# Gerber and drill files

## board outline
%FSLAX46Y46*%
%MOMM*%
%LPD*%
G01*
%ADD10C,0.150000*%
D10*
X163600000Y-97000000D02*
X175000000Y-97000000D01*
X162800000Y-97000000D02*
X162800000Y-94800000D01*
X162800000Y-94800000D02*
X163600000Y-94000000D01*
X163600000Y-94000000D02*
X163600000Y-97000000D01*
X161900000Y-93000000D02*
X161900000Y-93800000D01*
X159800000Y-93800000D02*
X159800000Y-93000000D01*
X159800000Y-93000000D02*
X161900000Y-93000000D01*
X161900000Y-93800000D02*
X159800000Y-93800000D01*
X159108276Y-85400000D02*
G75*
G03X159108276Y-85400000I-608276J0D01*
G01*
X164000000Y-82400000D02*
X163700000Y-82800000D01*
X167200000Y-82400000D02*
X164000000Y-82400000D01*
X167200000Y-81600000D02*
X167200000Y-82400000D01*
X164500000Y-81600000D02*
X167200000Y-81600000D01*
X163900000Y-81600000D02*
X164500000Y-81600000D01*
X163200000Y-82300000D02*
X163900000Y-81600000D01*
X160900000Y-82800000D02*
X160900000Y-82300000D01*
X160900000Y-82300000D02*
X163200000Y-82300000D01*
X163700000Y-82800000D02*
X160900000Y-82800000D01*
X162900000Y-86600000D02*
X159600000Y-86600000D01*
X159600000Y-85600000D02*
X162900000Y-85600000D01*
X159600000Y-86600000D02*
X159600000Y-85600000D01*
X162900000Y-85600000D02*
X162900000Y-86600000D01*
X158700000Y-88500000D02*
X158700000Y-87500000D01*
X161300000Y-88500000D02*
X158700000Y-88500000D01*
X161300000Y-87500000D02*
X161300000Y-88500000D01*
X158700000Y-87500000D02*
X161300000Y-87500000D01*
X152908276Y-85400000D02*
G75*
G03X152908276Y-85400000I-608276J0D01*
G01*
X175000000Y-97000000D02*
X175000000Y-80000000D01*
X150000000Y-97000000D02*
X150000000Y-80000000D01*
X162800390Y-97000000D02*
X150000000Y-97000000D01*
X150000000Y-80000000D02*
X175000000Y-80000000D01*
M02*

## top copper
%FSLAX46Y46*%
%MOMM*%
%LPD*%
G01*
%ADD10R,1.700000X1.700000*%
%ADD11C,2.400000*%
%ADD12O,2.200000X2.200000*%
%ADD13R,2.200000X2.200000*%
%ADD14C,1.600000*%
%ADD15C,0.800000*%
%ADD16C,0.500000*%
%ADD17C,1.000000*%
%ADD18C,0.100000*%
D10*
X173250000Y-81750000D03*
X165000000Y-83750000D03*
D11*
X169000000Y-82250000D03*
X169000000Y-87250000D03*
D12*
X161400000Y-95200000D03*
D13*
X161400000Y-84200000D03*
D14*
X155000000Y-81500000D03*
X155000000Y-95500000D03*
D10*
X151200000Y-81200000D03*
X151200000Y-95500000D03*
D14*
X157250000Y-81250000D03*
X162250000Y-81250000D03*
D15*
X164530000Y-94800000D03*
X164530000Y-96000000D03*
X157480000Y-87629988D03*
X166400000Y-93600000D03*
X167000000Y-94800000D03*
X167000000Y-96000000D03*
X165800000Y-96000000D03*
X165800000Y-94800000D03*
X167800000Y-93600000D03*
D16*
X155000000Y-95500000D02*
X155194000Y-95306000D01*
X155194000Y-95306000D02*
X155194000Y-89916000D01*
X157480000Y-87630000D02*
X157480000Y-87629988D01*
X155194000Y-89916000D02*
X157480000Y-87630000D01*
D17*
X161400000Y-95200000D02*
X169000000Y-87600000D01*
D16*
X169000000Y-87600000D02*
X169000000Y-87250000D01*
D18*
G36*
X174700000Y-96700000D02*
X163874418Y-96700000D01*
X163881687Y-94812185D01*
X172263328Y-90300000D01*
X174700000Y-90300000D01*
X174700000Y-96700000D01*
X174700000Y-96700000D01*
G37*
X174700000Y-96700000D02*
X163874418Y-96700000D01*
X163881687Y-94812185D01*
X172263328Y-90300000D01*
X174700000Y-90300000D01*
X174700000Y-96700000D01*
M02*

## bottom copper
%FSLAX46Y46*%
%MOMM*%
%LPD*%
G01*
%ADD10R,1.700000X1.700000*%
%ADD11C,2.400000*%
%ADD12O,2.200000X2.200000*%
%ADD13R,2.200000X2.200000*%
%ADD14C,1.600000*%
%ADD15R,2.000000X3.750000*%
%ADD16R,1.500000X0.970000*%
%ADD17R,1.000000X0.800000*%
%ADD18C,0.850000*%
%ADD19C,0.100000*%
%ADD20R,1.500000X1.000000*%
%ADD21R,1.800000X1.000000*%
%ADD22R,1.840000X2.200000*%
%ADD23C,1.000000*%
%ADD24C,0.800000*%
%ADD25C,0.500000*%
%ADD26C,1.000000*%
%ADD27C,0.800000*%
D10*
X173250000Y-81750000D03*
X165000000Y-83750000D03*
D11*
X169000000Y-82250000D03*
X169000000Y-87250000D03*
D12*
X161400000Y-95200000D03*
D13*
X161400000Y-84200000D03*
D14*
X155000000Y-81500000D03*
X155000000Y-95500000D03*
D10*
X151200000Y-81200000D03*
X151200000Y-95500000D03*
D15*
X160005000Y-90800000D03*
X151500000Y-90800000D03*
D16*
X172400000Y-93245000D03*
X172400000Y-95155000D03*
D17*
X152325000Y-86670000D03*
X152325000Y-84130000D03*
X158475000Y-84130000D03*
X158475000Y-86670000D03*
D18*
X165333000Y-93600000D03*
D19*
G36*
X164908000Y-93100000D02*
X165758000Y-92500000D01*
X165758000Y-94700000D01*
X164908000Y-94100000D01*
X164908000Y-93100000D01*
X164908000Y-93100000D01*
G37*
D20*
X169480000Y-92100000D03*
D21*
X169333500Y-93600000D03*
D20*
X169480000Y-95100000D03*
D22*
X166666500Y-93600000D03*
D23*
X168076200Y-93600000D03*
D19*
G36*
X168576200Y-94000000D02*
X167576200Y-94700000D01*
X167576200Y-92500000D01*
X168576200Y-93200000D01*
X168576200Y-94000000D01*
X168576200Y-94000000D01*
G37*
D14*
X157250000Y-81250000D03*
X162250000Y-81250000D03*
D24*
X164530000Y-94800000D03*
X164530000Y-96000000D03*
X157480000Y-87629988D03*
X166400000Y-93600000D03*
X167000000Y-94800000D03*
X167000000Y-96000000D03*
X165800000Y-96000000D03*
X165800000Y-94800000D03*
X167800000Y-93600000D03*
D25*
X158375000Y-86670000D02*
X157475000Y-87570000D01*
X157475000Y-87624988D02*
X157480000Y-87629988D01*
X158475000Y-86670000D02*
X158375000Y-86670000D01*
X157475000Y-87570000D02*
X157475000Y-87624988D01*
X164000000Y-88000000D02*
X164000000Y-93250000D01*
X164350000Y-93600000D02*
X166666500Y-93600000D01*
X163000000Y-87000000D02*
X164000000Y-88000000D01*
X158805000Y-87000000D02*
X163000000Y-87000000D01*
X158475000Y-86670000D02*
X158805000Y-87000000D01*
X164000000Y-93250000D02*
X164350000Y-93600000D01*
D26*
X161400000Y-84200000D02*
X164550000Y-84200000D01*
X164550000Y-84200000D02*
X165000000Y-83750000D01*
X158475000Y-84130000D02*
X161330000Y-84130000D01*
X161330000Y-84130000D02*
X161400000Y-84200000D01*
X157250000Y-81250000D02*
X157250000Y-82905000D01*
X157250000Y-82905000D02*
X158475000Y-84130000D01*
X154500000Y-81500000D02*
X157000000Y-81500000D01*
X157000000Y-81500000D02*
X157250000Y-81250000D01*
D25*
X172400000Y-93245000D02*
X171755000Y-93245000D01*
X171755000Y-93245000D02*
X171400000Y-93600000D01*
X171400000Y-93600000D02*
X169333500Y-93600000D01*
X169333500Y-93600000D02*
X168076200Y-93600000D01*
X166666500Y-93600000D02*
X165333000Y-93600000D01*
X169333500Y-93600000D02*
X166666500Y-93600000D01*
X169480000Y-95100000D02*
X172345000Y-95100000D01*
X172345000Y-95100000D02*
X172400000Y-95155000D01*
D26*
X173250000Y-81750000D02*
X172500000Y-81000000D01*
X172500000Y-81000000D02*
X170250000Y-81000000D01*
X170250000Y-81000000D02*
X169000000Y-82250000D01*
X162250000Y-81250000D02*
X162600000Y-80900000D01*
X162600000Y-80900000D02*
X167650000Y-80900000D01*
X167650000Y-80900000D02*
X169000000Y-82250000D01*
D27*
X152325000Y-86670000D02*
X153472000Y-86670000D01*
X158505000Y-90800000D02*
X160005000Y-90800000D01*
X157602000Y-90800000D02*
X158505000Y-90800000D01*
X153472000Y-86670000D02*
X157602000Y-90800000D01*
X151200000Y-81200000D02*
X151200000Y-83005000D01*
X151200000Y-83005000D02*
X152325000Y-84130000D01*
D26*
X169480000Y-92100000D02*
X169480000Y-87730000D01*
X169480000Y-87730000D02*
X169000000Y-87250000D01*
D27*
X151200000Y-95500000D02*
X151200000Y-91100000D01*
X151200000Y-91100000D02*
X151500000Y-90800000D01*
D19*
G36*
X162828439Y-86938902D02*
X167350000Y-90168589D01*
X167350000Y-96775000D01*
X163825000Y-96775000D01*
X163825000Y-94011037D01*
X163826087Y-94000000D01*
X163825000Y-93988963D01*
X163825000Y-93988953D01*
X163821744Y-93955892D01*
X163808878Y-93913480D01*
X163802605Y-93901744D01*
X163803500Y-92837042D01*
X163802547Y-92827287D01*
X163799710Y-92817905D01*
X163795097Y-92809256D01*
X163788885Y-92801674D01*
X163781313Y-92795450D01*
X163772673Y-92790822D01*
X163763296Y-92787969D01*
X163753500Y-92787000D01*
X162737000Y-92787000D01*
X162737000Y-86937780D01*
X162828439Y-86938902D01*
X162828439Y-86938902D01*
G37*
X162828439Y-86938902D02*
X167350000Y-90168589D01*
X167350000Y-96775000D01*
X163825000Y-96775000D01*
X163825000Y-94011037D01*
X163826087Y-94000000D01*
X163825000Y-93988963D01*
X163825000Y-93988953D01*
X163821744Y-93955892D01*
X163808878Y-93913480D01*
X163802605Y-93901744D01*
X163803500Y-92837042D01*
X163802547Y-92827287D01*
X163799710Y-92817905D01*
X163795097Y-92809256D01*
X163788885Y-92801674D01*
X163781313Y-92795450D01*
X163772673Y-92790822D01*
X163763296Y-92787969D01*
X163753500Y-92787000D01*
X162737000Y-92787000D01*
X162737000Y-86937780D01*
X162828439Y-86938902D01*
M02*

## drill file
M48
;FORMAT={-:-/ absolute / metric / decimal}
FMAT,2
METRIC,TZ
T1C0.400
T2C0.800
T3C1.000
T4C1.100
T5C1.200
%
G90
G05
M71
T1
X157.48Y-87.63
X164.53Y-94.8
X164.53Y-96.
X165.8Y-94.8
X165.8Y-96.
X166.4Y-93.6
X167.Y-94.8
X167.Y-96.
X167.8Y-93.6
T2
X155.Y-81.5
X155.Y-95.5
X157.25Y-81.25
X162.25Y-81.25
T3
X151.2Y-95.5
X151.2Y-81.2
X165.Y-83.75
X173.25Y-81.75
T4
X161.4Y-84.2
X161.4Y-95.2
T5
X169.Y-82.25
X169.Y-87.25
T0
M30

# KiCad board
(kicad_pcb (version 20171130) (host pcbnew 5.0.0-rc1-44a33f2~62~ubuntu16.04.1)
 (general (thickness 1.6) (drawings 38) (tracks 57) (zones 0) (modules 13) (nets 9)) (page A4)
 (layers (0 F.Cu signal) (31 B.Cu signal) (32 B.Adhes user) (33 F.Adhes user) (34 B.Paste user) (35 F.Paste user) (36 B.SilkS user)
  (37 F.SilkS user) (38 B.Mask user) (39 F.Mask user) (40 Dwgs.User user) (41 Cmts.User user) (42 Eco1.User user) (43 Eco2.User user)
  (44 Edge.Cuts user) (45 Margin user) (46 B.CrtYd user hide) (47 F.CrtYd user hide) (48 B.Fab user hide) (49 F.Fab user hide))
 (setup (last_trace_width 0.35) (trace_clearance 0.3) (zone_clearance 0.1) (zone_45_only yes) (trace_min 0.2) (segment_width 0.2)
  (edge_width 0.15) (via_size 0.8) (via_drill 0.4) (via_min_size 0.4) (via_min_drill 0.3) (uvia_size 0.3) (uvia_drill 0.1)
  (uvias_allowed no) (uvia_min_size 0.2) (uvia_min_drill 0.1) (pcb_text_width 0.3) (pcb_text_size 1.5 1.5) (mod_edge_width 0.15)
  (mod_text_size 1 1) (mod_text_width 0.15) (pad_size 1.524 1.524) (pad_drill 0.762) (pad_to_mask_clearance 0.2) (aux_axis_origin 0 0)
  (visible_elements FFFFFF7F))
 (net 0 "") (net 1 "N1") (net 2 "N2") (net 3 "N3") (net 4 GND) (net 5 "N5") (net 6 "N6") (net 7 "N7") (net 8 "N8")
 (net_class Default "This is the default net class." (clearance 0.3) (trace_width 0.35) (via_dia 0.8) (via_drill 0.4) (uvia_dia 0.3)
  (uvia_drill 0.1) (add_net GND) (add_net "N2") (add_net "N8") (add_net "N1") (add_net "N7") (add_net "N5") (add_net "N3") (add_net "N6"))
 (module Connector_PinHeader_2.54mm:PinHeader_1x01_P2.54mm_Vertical (layer F.Cu) (at 173.25 81.75)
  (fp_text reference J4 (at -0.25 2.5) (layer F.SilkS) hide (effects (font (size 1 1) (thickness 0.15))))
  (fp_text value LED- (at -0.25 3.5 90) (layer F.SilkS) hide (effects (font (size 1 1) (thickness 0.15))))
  (pad 1 thru_hole rect (at 0 0) (size 1.7 1.7) (drill 1) (layers *.Cu *.Mask) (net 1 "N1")))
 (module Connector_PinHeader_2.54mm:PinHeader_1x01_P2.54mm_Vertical (layer F.Cu) (at 165 83.75)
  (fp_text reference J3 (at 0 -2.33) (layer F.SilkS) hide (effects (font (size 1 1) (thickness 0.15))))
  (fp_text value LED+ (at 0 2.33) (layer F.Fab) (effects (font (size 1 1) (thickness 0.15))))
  (pad 1 thru_hole rect (at 0 0) (size 1.7 1.7) (drill 1) (layers *.Cu *.Mask) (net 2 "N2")))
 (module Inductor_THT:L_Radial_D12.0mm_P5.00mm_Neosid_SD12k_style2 (layer F.Cu) (at 169 82.25 270)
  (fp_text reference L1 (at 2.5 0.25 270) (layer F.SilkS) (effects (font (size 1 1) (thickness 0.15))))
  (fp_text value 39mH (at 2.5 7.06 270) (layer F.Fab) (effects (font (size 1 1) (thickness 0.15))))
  (pad 1 thru_hole circle (at 0 0 270) (size 2.4 2.4) (drill 1.2) (layers *.Cu *.Mask) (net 1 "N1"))
  (pad 2 thru_hole circle (at 5 0 270) (size 2.4 2.4) (drill 1.2) (layers *.Cu *.Mask) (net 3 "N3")))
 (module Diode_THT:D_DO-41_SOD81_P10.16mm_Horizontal (layer F.Cu) (at 161.4 84.2 270)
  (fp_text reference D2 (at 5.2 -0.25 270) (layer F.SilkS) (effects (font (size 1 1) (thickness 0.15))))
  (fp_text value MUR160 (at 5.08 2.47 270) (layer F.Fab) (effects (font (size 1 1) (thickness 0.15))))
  (pad 2 thru_hole oval (at 11 0 270) (size 2.2 2.2) (drill 1.1) (layers *.Cu *.Mask) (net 3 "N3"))
  (pad 1 thru_hole rect (at 0 0 270) (size 2.2 2.2) (drill 1.1) (layers *.Cu *.Mask) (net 2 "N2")))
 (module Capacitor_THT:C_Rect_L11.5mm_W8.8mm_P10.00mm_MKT (layer F.Cu) (at 155 83.5 270)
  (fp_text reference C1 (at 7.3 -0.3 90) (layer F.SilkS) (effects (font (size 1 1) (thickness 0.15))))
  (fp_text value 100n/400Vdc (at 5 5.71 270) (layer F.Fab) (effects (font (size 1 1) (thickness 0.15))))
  (pad 1 thru_hole circle (at -2 0 270) (size 1.6 1.6) (drill 0.8) (layers *.Cu *.Mask) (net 2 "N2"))
  (pad 2 thru_hole circle (at 12 0 270) (size 1.6 1.6) (drill 0.8) (layers *.Cu *.Mask) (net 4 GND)))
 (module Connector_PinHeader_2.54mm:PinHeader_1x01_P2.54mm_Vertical (layer F.Cu) (at 151.2 81.2)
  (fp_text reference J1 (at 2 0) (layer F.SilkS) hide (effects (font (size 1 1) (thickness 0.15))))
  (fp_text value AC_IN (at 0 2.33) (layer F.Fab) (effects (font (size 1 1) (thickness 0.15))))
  (pad 1 thru_hole rect (at 0 0) (size 1.7 1.7) (drill 1) (layers *.Cu *.Mask) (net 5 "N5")))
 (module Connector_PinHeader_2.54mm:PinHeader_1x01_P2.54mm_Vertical (layer F.Cu) (at 151.2 95.5)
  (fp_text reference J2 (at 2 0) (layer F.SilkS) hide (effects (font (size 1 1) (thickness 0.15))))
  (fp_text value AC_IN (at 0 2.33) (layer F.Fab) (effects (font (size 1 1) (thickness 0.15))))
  (pad 1 thru_hole rect (at 0 0) (size 1.7 1.7) (drill 1) (layers *.Cu *.Mask) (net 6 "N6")))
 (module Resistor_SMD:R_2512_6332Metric (layer B.Cu) (at 157 90.8 180)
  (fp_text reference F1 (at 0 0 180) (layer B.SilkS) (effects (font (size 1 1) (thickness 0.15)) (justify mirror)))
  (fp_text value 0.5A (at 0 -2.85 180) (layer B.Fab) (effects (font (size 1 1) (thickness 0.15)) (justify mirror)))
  (pad 1 smd rect (at -3.005 0 180) (size 2 3.75) (layers B.Cu B.Paste B.Mask) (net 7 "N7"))
  (pad 2 smd rect (at 5.5 0 180) (size 2 3.75) (layers B.Cu B.Paste B.Mask) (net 6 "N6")))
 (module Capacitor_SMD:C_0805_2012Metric (layer B.Cu) (at 172.4 94.2 270)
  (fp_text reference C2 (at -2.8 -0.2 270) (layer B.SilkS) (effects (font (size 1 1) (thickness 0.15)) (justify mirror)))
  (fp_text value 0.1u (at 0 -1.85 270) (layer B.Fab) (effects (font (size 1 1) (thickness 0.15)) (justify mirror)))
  (pad 1 smd rect (at -0.955 0 270) (size 0.97 1.5) (layers B.Cu B.Paste B.Mask) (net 4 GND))
  (pad 2 smd rect (at 0.955 0 270) (size 0.97 1.5) (layers B.Cu B.Paste B.Mask) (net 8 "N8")))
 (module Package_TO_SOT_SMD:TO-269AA (layer B.Cu) (at 155.4 85.4)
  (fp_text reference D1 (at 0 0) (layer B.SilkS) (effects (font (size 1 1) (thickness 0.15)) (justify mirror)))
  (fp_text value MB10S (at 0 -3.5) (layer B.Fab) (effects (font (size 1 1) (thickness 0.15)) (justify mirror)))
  (pad 1 smd rect (at -3.075 1.27) (size 1 0.8) (layers B.Cu B.Paste B.Mask) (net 7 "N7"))
  (pad 2 smd rect (at -3.075 -1.27) (size 1 0.8) (layers B.Cu B.Paste B.Mask) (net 5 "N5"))
  (pad 3 smd rect (at 3.075 -1.27) (size 1 0.8) (layers B.Cu B.Paste B.Mask) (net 2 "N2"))
  (pad 4 smd rect (at 3.075 1.27) (size 1 0.8) (layers B.Cu B.Paste B.Mask) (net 4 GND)))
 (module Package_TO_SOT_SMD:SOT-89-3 (layer B.Cu) (at 168 93.6 180)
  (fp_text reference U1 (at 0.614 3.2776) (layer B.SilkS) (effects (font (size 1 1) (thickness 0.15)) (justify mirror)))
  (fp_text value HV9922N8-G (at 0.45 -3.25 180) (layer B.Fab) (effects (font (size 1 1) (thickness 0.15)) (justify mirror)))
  (pad 2 smd trapezoid (at 2.667 0 270) (size 1.6 0.85) (rect_delta 0 -0.6) (layers B.Cu B.Paste B.Mask) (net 4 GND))
  (pad 1 smd rect (at -1.48 1.5 270) (size 1 1.5) (layers B.Cu B.Paste B.Mask) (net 3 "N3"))
  (pad 2 smd rect (at -1.3335 0 270) (size 1 1.8) (layers B.Cu B.Paste B.Mask) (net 4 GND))
  (pad 3 smd rect (at -1.48 -1.5 270) (size 1 1.5) (layers B.Cu B.Paste B.Mask) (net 8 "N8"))
  (pad 2 smd rect (at 1.3335 0 270) (size 2.2 1.84) (layers B.Cu B.Paste B.Mask) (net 4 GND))
  (pad 2 smd trapezoid (at -0.0762 0 90) (size 1.5 1) (rect_delta 0 -0.7) (layers B.Cu B.Paste B.Mask) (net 4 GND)))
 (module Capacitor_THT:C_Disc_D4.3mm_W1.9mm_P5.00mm (layer F.Cu) (at 157.25 81.25)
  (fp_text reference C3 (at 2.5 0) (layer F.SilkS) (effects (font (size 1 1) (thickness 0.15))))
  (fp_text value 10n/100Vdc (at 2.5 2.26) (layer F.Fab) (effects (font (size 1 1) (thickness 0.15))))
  (pad 1 thru_hole circle (at 0 0) (size 1.6 1.6) (drill 0.8) (layers *.Cu *.Mask) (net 2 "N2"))
  (pad 2 thru_hole circle (at 5 0) (size 1.6 1.6) (drill 0.8) (layers *.Cu *.Mask) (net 1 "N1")))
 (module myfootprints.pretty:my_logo (layer F.Cu) (at 170.942 93.98)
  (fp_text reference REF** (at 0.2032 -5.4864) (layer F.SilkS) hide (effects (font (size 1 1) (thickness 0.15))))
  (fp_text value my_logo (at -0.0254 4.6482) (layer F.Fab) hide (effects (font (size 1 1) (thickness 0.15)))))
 (gr_line (start 163.6 97) (end 175 97) (layer Edge.Cuts) (width 0.15))
 (gr_line (start 162.8 97) (end 162.8 94.8) (layer Edge.Cuts) (width 0.15))
 (gr_line (start 162.8 94.8) (end 163.6 94) (layer Edge.Cuts) (width 0.15))
 (gr_line (start 163.6 94) (end 163.6 97) (layer Edge.Cuts) (width 0.15))
 (gr_line (start 161.9 93) (end 161.9 93.8) (layer Edge.Cuts) (width 0.15))
 (gr_line (start 159.8 93.8) (end 159.8 93) (layer Edge.Cuts) (width 0.15))
 (gr_line (start 159.8 93) (end 161.9 93) (layer Edge.Cuts) (width 0.15))
 (gr_line (start 161.9 93.8) (end 159.8 93.8) (layer Edge.Cuts) (width 0.15))
 (gr_circle (center 158.5 85.4) (end 159.108276 85.4) (layer Edge.Cuts) (width 0.15))
 (gr_line (start 164 82.4) (end 163.7 82.8) (layer Edge.Cuts) (width 0.15))
 (gr_line (start 167.2 82.4) (end 164 82.4) (layer Edge.Cuts) (width 0.15))
 (gr_line (start 167.2 81.6) (end 167.2 82.4) (layer Edge.Cuts) (width 0.15))
 (gr_line (start 164.5 81.6) (end 167.2 81.6) (layer Edge.Cuts) (width 0.15))
 (gr_line (start 163.9 81.6) (end 164.5 81.6) (layer Edge.Cuts) (width 0.15))
 (gr_line (start 163.2 82.3) (end 163.9 81.6) (layer Edge.Cuts) (width 0.15))
 (gr_line (start 160.9 82.8) (end 160.9 82.3) (layer Edge.Cuts) (width 0.15))
 (gr_line (start 160.9 82.3) (end 163.2 82.3) (layer Edge.Cuts) (width 0.15))
 (gr_line (start 163.7 82.8) (end 160.9 82.8) (layer Edge.Cuts) (width 0.15))
 (gr_line (start 162.9 86.6) (end 159.6 86.6) (layer Edge.Cuts) (width 0.15))
 (gr_line (start 159.6 85.6) (end 162.9 85.6) (layer Edge.Cuts) (width 0.15))
 (gr_line (start 159.6 86.6) (end 159.6 85.6) (layer Edge.Cuts) (width 0.15))
 (gr_line (start 162.9 85.6) (end 162.9 86.6) (layer Edge.Cuts) (width 0.15))
 (gr_line (start 158.7 88.5) (end 158.7 87.5) (layer Edge.Cuts) (width 0.15))
 (gr_line (start 161.3 88.5) (end 158.7 88.5) (layer Edge.Cuts) (width 0.15))
 (gr_line (start 161.3 87.5) (end 161.3 88.5) (layer Edge.Cuts) (width 0.15))
 (gr_line (start 158.7 87.5) (end 161.3 87.5) (layer Edge.Cuts) (width 0.15))
 (gr_circle (center 152.3 85.4) (end 152.908276 85.4) (layer Edge.Cuts) (width 0.15))
 (gr_line (start 175 97) (end 175 80) (layer Edge.Cuts) (width 0.15))
 (gr_line (start 150 97) (end 150 80) (layer Edge.Cuts) (width 0.15))
 (gr_line (start 162.80039 97) (end 150 97) (layer Edge.Cuts) (width 0.15))
 (gr_line (start 150 80) (end 175 80) (layer Edge.Cuts) (width 0.15))
 (via (at 164.53 94.8) (size 0.8) (drill 0.4) (layers F.Cu B.Cu) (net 4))
 (via (at 164.53 96) (size 0.8) (drill 0.4) (layers F.Cu B.Cu) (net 4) (status 1000000))
 (segment (start 155 95.5) (end 155.194 95.306) (width 0.5) (layer F.Cu) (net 4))
 (segment (start 155.194 95.306) (end 155.194 89.916) (width 0.5) (layer F.Cu) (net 4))
 (segment (start 157.48 87.63) (end 157.48 87.629988) (width 0.5) (layer F.Cu) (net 4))
 (segment (start 155.194 89.916) (end 157.48 87.63) (width 0.5) (layer F.Cu) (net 4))
 (segment (start 158.375 86.67) (end 157.475 87.57) (width 0.5) (layer B.Cu) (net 4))
 (segment (start 157.475 87.624988) (end 157.48 87.629988) (width 0.5) (layer B.Cu) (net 4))
 (segment (start 158.475 86.67) (end 158.375 86.67) (width 0.5) (layer B.Cu) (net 4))
 (segment (start 157.475 87.57) (end 157.475 87.624988) (width 0.5) (layer B.Cu) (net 4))
 (via (at 157.48 87.629988) (size 0.8) (drill 0.4) (layers F.Cu B.Cu) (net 4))
 (segment (start 164 88) (end 164 93.25) (width 0.5) (layer B.Cu) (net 4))
 (segment (start 164.35 93.6) (end 166.6665 93.6) (width 0.5) (layer B.Cu) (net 4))
 (segment (start 163 87) (end 164 88) (width 0.5) (layer B.Cu) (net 4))
 (segment (start 158.805 87) (end 163 87) (width 0.5) (layer B.Cu) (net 4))
 (segment (start 158.475 86.67) (end 158.805 87) (width 0.5) (layer B.Cu) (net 4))
 (segment (start 164 93.25) (end 164.35 93.6) (width 0.5) (layer B.Cu) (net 4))
 (via (at 166.4 93.6) (size 0.8) (drill 0.4) (layers F.Cu B.Cu) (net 4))
 (via (at 167 94.8) (size 0.8) (drill 0.4) (layers F.Cu B.Cu) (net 4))
 (via (at 167 96) (size 0.8) (drill 0.4) (layers F.Cu B.Cu) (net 4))
 (via (at 165.8 96) (size 0.8) (drill 0.4) (layers F.Cu B.Cu) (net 4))
 (via (at 165.8 94.8) (size 0.8) (drill 0.4) (layers F.Cu B.Cu) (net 4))
 (via (at 167.8 93.6) (size 0.8) (drill 0.4) (layers F.Cu B.Cu) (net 4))
 (segment (start 161.4 84.2) (end 164.55 84.2) (width 1) (layer B.Cu) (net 2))
 (segment (start 164.55 84.2) (end 165 83.75) (width 1) (layer B.Cu) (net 2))
 (segment (start 158.475 84.13) (end 161.33 84.13) (width 1) (layer B.Cu) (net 2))
 (segment (start 161.33 84.13) (end 161.4 84.2) (width 1) (layer B.Cu) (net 2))
 (segment (start 157.25 81.25) (end 157.25 82.905) (width 1) (layer B.Cu) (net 2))
 (segment (start 157.25 82.905) (end 158.475 84.13) (width 1) (layer B.Cu) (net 2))
 (segment (start 154.5 81.5) (end 157 81.5) (width 1) (layer B.Cu) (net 2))
 (segment (start 157 81.5) (end 157.25 81.25) (width 1) (layer B.Cu) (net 2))
 (segment (start 172.4 93.245) (end 171.755 93.245) (width 0.5) (layer B.Cu) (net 4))
 (segment (start 171.755 93.245) (end 171.4 93.6) (width 0.5) (layer B.Cu) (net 4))
 (segment (start 171.4 93.6) (end 169.3335 93.6) (width 0.5) (layer B.Cu) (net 4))
 (segment (start 169.3335 93.6) (end 168.0762 93.6) (width 0.5) (layer B.Cu) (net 4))
 (segment (start 166.6665 93.6) (end 165.333 93.6) (width 0.5) (layer B.Cu) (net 4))
 (segment (start 169.3335 93.6) (end 166.6665 93.6) (width 0.5) (layer B.Cu) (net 4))
 (segment (start 169.48 95.1) (end 172.345 95.1) (width 0.5) (layer B.Cu) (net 8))
 (segment (start 172.345 95.1) (end 172.4 95.155) (width 0.5) (layer B.Cu) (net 8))
 (segment (start 173.25 81.75) (end 172.5 81) (width 1) (layer B.Cu) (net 1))
 (segment (start 172.5 81) (end 170.25 81) (width 1) (layer B.Cu) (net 1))
 (segment (start 170.25 81) (end 169 82.25) (width 1) (layer B.Cu) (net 1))
 (segment (start 162.25 81.25) (end 162.6 80.9) (width 1) (layer B.Cu) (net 1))
 (segment (start 162.6 80.9) (end 167.65 80.9) (width 1) (layer B.Cu) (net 1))
 (segment (start 167.65 80.9) (end 169 82.25) (width 1) (layer B.Cu) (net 1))
 (segment (start 152.325 86.67) (end 153.472 86.67) (width 0.8) (layer B.Cu) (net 7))
 (segment (start 158.505 90.8) (end 160.005 90.8) (width 0.8) (layer B.Cu) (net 7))
 (segment (start 157.602 90.8) (end 158.505 90.8) (width 0.8) (layer B.Cu) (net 7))
 (segment (start 153.472 86.67) (end 157.602 90.8) (width 0.8) (layer B.Cu) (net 7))
 (segment (start 151.2 81.2) (end 151.2 83.005) (width 0.8) (layer B.Cu) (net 5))
 (segment (start 151.2 83.005) (end 152.325 84.13) (width 0.8) (layer B.Cu) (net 5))
 (segment (start 169.48 92.1) (end 169.48 87.73) (width 1) (layer B.Cu) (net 3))
 (segment (start 169.48 87.73) (end 169 87.25) (width 1) (layer B.Cu) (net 3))
 (segment (start 161.4 95.2) (end 169 87.6) (width 1) (layer F.Cu) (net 3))
 (segment (start 169 87.6) (end 169 87.25) (width 0.5) (layer F.Cu) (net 3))
 (segment (start 151.2 95.5) (end 151.2 91.1) (width 0.8) (layer B.Cu) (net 6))
 (segment (start 151.2 91.1) (end 151.5 90.8) (width 0.8) (layer B.Cu) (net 6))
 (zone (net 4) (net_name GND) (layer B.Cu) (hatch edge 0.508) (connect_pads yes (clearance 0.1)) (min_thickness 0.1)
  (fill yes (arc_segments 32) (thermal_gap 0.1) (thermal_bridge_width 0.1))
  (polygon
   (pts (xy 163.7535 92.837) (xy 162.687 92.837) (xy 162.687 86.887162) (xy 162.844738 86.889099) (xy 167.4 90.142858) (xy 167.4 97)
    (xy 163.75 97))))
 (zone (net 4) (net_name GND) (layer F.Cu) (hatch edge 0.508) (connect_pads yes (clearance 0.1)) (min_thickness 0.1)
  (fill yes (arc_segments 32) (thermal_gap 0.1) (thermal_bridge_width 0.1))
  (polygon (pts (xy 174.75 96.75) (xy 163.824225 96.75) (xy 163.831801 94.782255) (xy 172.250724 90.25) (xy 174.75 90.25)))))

